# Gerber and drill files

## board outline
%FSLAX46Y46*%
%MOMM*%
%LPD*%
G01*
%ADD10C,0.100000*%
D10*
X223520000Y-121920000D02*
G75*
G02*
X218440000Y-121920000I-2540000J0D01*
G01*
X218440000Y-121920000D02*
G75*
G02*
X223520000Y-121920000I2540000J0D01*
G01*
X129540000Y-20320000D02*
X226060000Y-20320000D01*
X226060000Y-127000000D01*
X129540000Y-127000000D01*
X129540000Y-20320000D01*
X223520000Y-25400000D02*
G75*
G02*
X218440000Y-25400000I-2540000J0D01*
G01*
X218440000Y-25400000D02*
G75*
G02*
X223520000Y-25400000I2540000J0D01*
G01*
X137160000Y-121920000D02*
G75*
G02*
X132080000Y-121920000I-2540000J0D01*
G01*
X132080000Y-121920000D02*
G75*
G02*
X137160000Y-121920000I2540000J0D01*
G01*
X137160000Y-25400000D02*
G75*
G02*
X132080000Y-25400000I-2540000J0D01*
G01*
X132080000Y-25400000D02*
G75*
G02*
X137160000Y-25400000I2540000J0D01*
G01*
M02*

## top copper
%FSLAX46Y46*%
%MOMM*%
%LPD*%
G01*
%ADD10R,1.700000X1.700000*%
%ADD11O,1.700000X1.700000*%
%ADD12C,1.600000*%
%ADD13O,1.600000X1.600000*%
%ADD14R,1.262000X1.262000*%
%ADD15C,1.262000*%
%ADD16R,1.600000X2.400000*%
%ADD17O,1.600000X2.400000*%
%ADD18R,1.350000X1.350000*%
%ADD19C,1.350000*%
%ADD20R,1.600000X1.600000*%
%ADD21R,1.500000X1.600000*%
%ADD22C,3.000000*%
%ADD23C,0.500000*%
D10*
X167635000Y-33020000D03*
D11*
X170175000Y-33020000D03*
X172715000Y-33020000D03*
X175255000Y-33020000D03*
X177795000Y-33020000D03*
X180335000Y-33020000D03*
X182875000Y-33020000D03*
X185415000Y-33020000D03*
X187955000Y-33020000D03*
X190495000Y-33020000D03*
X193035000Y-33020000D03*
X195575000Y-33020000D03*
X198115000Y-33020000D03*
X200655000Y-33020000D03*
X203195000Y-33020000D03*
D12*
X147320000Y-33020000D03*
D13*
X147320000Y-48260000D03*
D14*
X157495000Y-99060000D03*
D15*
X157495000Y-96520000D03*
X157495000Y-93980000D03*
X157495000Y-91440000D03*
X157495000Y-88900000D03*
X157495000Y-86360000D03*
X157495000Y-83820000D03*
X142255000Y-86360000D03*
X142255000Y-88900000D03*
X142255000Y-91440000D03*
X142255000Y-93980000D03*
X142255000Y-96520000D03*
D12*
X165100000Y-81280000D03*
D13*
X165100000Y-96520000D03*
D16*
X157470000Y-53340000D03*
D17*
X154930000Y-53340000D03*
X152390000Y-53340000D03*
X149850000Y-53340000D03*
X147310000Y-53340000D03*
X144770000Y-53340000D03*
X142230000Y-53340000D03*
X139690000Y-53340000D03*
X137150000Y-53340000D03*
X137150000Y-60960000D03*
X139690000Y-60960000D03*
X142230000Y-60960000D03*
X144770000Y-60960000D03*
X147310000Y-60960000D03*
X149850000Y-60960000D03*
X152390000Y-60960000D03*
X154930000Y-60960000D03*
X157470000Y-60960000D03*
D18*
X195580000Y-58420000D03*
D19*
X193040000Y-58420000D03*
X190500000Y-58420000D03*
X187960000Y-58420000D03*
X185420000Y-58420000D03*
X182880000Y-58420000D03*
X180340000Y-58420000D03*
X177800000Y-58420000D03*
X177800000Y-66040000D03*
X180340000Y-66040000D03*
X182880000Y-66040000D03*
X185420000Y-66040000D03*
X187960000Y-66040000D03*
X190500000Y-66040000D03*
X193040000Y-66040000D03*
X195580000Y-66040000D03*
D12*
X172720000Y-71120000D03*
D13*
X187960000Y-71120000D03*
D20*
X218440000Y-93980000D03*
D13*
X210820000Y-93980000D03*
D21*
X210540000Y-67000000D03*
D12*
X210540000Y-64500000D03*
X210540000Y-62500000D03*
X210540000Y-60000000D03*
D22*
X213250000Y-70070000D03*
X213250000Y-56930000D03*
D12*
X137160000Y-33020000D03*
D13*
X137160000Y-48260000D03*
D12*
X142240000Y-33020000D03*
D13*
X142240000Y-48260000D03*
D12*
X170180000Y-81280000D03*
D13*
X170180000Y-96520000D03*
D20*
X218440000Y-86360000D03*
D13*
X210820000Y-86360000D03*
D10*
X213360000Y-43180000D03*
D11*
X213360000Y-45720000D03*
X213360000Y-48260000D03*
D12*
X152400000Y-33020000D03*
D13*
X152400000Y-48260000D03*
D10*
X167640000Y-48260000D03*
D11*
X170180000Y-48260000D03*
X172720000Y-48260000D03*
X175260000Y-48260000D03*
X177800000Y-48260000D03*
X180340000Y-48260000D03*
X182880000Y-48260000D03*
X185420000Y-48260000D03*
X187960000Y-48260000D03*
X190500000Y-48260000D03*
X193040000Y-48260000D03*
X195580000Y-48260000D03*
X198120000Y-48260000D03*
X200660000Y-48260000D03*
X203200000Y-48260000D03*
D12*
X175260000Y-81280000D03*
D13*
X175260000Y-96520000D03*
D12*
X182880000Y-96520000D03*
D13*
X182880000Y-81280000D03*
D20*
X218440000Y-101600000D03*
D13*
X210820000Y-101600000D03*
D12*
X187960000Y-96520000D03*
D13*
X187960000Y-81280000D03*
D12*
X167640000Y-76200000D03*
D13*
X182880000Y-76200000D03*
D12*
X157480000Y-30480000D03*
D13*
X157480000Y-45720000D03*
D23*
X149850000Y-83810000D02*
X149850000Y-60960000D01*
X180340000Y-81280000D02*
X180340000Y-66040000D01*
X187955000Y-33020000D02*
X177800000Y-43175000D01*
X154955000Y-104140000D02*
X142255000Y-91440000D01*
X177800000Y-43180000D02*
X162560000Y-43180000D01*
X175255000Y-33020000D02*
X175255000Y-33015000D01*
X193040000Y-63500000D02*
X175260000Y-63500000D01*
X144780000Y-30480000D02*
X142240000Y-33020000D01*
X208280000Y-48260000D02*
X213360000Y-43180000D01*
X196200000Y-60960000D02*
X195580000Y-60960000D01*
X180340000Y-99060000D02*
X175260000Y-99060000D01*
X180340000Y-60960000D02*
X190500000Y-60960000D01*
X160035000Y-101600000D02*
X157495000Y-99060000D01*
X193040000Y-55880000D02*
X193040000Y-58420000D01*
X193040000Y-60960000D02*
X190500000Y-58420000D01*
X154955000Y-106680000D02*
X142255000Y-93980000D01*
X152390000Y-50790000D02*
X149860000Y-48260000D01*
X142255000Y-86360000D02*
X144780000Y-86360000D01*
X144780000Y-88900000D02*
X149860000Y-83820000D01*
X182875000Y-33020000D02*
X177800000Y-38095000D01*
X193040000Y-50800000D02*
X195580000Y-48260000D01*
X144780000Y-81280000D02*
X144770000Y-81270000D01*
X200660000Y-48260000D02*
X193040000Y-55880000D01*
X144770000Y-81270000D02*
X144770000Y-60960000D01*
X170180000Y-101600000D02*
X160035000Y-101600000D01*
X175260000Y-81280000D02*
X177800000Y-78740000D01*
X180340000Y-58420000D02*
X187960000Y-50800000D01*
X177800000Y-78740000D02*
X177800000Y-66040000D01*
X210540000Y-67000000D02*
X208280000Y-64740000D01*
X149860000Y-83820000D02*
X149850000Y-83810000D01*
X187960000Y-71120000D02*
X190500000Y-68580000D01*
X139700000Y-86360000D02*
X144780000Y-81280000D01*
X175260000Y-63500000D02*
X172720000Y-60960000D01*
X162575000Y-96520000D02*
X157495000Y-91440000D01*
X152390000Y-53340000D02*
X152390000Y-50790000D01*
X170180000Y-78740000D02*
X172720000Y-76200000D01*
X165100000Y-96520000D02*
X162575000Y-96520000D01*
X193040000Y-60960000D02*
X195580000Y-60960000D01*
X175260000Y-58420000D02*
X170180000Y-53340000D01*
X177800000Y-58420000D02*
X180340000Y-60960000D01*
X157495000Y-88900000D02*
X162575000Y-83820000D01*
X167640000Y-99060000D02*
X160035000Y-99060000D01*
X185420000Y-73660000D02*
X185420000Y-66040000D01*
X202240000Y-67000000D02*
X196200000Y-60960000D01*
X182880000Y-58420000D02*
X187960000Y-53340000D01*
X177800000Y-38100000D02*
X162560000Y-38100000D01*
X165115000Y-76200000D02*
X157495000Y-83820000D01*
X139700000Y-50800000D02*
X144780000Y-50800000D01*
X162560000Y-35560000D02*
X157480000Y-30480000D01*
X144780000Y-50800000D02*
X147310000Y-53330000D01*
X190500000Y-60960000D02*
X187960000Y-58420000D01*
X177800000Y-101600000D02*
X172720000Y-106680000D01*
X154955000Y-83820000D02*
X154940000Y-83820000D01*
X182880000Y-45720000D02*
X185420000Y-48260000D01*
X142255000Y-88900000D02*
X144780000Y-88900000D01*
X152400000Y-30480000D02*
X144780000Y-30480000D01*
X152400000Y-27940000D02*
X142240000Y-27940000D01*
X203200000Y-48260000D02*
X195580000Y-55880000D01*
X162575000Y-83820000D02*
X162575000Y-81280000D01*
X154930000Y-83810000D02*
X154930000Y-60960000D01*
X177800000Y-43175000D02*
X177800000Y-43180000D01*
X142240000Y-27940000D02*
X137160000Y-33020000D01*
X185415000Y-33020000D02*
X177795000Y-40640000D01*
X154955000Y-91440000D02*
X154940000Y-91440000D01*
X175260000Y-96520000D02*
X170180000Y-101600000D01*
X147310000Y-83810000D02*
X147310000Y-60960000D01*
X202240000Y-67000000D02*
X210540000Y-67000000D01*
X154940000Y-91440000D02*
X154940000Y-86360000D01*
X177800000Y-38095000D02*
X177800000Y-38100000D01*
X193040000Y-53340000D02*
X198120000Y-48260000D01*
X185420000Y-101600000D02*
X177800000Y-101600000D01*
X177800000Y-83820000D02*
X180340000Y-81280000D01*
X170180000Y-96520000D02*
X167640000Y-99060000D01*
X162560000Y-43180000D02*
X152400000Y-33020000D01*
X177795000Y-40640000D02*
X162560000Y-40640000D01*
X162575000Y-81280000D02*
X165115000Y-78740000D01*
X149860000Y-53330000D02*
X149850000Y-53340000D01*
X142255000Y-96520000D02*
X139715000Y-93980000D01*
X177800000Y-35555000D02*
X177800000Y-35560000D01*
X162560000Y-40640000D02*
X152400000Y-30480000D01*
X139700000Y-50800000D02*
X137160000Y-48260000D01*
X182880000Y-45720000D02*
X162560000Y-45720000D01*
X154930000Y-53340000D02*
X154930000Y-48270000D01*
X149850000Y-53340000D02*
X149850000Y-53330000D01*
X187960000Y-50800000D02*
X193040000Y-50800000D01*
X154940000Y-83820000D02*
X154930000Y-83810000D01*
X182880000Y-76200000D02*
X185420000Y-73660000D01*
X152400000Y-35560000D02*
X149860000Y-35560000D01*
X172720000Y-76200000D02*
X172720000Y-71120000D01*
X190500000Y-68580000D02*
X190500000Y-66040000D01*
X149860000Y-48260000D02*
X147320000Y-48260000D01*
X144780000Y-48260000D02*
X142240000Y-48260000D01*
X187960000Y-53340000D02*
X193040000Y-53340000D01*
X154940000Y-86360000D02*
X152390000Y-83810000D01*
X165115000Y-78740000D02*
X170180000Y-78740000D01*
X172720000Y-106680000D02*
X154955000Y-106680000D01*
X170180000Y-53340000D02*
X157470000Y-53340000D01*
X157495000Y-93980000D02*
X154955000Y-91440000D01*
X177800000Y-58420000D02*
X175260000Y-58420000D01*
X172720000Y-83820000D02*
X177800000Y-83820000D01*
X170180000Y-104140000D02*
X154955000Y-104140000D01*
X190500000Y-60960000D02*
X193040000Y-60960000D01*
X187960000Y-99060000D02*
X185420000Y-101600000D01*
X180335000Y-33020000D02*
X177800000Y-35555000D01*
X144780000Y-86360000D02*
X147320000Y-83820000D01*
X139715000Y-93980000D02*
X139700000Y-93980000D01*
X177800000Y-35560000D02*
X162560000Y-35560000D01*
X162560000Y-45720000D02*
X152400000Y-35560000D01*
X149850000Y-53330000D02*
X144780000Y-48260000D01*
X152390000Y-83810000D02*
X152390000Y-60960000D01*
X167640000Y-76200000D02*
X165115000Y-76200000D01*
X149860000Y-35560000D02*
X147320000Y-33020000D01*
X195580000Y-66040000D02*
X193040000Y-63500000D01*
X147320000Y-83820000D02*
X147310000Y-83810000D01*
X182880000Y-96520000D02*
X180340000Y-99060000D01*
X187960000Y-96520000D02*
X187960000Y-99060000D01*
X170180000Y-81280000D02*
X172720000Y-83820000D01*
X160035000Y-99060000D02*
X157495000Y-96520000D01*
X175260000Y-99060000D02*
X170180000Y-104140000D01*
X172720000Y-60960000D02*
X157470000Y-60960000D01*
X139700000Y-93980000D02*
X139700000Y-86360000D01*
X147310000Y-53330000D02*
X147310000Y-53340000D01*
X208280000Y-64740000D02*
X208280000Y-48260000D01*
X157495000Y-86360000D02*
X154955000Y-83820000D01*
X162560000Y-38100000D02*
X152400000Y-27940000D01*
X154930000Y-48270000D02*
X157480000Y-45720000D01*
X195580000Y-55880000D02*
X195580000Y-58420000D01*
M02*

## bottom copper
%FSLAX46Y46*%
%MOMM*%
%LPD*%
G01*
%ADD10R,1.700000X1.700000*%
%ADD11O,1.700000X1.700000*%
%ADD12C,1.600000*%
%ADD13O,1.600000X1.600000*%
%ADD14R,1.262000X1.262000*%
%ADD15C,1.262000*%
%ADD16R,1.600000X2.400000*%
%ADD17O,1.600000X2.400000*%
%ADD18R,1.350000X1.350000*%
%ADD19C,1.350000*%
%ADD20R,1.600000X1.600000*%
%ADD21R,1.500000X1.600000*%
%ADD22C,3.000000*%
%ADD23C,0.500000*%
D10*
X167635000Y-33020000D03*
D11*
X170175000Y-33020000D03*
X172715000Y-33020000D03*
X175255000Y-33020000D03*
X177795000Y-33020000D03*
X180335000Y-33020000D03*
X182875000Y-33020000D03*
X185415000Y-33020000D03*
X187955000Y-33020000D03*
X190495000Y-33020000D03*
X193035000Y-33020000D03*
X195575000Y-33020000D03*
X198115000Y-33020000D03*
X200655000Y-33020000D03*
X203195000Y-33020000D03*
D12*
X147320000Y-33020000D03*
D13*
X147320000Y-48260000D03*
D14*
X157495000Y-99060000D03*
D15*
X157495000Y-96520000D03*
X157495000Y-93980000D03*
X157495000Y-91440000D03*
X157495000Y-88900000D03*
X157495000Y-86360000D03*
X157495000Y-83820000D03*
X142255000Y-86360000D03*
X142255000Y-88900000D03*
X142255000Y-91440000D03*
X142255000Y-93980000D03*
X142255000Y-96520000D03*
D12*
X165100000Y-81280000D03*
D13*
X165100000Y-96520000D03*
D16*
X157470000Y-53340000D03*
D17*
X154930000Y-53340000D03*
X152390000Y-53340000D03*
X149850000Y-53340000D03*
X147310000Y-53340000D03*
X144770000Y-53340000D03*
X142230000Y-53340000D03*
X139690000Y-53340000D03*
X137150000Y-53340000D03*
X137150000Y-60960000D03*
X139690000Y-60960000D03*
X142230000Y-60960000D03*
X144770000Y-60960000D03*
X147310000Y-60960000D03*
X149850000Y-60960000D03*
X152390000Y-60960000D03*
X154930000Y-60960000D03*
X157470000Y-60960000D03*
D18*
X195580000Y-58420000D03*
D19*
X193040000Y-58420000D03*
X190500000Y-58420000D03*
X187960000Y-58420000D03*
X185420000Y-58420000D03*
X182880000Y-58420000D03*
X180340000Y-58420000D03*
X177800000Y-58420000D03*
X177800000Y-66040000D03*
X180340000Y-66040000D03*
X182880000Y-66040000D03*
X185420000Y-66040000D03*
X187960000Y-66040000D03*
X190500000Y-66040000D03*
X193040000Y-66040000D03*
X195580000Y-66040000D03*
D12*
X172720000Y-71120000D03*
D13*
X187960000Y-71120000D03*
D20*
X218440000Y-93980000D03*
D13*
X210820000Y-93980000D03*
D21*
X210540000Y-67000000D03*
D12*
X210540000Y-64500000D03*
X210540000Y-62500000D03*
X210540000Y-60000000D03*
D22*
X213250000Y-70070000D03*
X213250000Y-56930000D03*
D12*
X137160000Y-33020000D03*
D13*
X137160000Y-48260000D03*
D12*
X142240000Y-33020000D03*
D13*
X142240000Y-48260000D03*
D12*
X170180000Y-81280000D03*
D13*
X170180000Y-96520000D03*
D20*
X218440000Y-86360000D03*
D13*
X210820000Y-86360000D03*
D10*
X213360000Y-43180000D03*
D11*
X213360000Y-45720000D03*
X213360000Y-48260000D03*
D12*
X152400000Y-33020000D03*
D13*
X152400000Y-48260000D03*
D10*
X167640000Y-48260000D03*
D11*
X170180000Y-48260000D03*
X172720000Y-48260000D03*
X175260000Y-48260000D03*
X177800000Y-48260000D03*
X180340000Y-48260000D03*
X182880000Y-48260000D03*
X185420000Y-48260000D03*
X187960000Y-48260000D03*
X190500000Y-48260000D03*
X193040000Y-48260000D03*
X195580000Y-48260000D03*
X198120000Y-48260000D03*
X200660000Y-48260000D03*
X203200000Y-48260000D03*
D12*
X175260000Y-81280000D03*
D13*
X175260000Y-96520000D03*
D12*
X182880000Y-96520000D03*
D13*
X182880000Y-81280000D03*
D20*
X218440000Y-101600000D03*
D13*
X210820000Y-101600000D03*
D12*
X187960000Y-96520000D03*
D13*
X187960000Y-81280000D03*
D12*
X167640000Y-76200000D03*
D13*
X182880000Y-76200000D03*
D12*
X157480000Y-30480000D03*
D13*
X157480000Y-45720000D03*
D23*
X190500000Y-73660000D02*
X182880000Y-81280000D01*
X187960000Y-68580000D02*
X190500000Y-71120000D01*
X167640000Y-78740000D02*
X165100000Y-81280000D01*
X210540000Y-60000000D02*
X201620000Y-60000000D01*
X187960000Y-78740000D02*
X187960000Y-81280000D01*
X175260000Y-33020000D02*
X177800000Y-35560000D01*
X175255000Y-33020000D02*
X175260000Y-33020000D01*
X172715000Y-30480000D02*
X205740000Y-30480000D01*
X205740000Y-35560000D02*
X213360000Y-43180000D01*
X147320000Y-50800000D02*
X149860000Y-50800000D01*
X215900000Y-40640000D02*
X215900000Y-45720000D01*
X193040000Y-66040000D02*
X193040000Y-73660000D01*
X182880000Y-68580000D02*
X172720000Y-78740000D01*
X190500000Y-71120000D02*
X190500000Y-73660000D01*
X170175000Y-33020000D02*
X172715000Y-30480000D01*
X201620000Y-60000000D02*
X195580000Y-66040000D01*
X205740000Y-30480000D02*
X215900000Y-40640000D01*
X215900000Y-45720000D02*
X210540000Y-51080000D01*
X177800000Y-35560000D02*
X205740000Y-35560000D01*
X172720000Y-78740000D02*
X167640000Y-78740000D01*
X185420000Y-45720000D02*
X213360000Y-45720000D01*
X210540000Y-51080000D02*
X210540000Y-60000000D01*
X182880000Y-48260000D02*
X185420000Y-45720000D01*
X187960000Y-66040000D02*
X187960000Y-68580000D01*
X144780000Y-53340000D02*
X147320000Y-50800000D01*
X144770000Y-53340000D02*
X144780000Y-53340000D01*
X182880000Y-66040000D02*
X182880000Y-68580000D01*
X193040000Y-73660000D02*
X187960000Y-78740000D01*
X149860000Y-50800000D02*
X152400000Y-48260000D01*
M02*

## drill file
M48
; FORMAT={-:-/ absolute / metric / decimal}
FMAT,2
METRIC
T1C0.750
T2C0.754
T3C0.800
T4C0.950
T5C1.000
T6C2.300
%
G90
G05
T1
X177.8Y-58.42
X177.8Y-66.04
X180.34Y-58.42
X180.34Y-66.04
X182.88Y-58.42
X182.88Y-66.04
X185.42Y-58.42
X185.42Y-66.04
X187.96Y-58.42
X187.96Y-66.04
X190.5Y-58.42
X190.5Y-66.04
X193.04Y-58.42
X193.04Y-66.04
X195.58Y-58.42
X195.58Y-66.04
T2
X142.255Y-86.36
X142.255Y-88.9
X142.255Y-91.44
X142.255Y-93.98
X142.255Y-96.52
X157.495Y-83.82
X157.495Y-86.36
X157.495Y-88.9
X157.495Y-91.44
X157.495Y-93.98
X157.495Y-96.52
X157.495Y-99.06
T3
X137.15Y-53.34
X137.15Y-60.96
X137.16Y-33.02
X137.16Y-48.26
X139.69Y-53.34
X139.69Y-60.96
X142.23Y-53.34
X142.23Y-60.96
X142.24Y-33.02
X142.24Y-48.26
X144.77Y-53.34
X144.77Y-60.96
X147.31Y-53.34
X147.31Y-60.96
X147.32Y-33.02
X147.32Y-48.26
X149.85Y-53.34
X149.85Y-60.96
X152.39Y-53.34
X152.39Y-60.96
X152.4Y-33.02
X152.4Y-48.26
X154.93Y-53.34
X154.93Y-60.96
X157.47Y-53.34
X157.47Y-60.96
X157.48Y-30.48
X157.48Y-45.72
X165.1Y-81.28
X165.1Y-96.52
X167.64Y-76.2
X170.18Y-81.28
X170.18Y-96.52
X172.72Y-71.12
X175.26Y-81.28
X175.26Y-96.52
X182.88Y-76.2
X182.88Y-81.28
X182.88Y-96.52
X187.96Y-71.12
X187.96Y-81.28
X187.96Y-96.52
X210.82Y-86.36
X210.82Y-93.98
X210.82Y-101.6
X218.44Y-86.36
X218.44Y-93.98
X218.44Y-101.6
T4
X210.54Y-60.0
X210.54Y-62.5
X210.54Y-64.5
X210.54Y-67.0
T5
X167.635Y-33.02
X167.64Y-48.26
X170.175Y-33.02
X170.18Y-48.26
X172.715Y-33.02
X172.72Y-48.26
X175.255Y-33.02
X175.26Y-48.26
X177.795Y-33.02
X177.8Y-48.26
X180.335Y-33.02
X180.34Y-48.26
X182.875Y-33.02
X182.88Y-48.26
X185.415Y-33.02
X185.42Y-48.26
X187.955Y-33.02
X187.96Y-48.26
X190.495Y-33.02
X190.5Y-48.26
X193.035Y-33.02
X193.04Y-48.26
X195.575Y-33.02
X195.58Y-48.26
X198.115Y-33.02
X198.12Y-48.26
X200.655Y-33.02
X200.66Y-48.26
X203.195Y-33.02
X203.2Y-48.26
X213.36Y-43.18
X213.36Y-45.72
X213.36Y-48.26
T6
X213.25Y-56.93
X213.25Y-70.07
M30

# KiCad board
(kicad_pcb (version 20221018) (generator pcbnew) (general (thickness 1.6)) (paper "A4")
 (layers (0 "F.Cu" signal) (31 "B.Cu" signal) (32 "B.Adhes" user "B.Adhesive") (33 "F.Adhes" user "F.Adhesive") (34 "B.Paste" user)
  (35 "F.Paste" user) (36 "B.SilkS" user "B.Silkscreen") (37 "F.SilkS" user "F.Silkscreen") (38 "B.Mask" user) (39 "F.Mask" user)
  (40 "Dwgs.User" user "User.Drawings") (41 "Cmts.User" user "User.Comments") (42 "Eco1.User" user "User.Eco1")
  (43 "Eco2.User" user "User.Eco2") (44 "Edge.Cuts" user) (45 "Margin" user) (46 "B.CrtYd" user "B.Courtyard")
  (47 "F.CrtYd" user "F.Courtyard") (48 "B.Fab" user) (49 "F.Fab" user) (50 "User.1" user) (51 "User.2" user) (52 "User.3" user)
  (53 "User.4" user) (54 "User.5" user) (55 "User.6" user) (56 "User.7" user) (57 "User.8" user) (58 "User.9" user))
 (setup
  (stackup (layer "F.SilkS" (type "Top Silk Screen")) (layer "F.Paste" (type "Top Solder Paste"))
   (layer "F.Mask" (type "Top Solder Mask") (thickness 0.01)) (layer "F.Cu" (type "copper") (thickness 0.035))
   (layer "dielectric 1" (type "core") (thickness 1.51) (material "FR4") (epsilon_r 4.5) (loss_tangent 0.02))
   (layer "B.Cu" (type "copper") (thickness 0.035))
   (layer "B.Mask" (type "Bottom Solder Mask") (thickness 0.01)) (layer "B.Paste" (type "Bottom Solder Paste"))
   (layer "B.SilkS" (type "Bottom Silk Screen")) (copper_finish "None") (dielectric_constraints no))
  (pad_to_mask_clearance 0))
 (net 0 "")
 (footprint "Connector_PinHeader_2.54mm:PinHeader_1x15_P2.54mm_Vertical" (layer "F.Cu") (at 167.635 33.02 90)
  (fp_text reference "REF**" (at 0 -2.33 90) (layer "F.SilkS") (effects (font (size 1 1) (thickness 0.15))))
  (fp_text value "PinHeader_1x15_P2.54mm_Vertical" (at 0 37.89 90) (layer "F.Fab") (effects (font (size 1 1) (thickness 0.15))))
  (pad "1" thru_hole rect (at 0 0 90) (size 1.7 1.7) (drill 1) (layers "*.Cu" "*.Mask"))
  (pad "2" thru_hole oval (at 0 2.54 90) (size 1.7 1.7) (drill 1) (layers "*.Cu" "*.Mask"))
  (pad "3" thru_hole oval (at 0 5.08 90) (size 1.7 1.7) (drill 1) (layers "*.Cu" "*.Mask"))
  (pad "4" thru_hole oval (at 0 7.62 90) (size 1.7 1.7) (drill 1) (layers "*.Cu" "*.Mask"))
  (pad "5" thru_hole oval (at 0 10.16 90) (size 1.7 1.7) (drill 1) (layers "*.Cu" "*.Mask"))
  (pad "6" thru_hole oval (at 0 12.7 90) (size 1.7 1.7) (drill 1) (layers "*.Cu" "*.Mask"))
  (pad "7" thru_hole oval (at 0 15.24 90) (size 1.7 1.7) (drill 1) (layers "*.Cu" "*.Mask"))
  (pad "8" thru_hole oval (at 0 17.78 90) (size 1.7 1.7) (drill 1) (layers "*.Cu" "*.Mask"))
  (pad "9" thru_hole oval (at 0 20.32 90) (size 1.7 1.7) (drill 1) (layers "*.Cu" "*.Mask"))
  (pad "10" thru_hole oval (at 0 22.86 90) (size 1.7 1.7) (drill 1) (layers "*.Cu" "*.Mask"))
  (pad "11" thru_hole oval (at 0 25.4 90) (size 1.7 1.7) (drill 1) (layers "*.Cu" "*.Mask"))
  (pad "12" thru_hole oval (at 0 27.94 90) (size 1.7 1.7) (drill 1) (layers "*.Cu" "*.Mask"))
  (pad "13" thru_hole oval (at 0 30.48 90) (size 1.7 1.7) (drill 1) (layers "*.Cu" "*.Mask"))
  (pad "14" thru_hole oval (at 0 33.02 90) (size 1.7 1.7) (drill 1) (layers "*.Cu" "*.Mask"))
  (pad "15" thru_hole oval (at 0 35.56 90) (size 1.7 1.7) (drill 1) (layers "*.Cu" "*.Mask")))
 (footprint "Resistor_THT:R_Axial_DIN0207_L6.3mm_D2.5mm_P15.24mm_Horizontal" (layer "F.Cu") (at 147.32 33.02 -90)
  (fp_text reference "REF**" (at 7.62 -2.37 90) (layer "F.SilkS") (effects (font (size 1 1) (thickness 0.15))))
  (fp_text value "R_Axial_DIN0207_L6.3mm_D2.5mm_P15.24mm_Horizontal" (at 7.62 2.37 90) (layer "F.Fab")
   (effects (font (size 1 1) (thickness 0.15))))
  (pad "1" thru_hole circle (at 0 0 270) (size 1.6 1.6) (drill 0.8) (layers "*.Cu" "*.Mask"))
  (pad "2" thru_hole oval (at 15.24 0 270) (size 1.6 1.6) (drill 0.8) (layers "*.Cu" "*.Mask")))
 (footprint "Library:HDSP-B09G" (layer "F.Cu") (at 149.875 91.44 90)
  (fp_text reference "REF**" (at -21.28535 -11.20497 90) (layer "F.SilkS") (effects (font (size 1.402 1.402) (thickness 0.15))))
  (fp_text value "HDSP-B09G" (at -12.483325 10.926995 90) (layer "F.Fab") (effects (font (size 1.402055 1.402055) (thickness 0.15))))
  (pad "1" thru_hole rect (at -7.62 7.62 90) (size 1.262 1.262) (drill 0.754) (layers "*.Cu" "*.Mask"))
  (pad "2" thru_hole circle (at -5.08 7.62 90) (size 1.262 1.262) (drill 0.754) (layers "*.Cu" "*.Mask"))
  (pad "3" thru_hole circle (at -2.54 7.62 90) (size 1.262 1.262) (drill 0.754) (layers "*.Cu" "*.Mask"))
  (pad "4" thru_hole circle (at 0 7.62 90) (size 1.262 1.262) (drill 0.754) (layers "*.Cu" "*.Mask"))
  (pad "5" thru_hole circle (at 2.54 7.62 90) (size 1.262 1.262) (drill 0.754) (layers "*.Cu" "*.Mask"))
  (pad "6" thru_hole circle (at 5.08 7.62 90) (size 1.262 1.262) (drill 0.754) (layers "*.Cu" "*.Mask"))
  (pad "7" thru_hole circle (at 7.62 7.62 90) (size 1.262 1.262) (drill 0.754) (layers "*.Cu" "*.Mask"))
  (pad "8" thru_hole circle (at 5.08 -7.62 90) (size 1.262 1.262) (drill 0.754) (layers "*.Cu" "*.Mask"))
  (pad "9" thru_hole circle (at 2.54 -7.62 90) (size 1.262 1.262) (drill 0.754) (layers "*.Cu" "*.Mask"))
  (pad "10" thru_hole circle (at 0 -7.62 90) (size 1.262 1.262) (drill 0.754) (layers "*.Cu" "*.Mask"))
  (pad "11" thru_hole circle (at -2.54 -7.62 90) (size 1.262 1.262) (drill 0.754) (layers "*.Cu" "*.Mask"))
  (pad "12" thru_hole circle (at -5.08 -7.62 90) (size 1.262 1.262) (drill 0.754) (layers "*.Cu" "*.Mask")))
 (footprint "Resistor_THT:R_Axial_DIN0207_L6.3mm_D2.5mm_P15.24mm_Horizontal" (layer "F.Cu") (at 165.1 81.28 -90)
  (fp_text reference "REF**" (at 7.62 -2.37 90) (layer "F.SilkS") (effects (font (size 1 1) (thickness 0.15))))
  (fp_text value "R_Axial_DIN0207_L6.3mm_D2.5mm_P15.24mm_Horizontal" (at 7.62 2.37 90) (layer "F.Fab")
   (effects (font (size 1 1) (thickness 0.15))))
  (pad "1" thru_hole circle (at 0 0 270) (size 1.6 1.6) (drill 0.8) (layers "*.Cu" "*.Mask"))
  (pad "2" thru_hole oval (at 15.24 0 270) (size 1.6 1.6) (drill 0.8) (layers "*.Cu" "*.Mask")))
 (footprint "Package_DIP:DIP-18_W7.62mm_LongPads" (layer "F.Cu") (at 157.47 53.34 -90)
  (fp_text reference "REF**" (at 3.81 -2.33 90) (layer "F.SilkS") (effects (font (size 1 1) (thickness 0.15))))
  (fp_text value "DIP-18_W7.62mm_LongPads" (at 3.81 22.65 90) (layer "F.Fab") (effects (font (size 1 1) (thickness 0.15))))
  (pad "1" thru_hole rect (at 0 0 270) (size 2.4 1.6) (drill 0.8) (layers "*.Cu" "*.Mask"))
  (pad "2" thru_hole oval (at 0 2.54 270) (size 2.4 1.6) (drill 0.8) (layers "*.Cu" "*.Mask"))
  (pad "3" thru_hole oval (at 0 5.08 270) (size 2.4 1.6) (drill 0.8) (layers "*.Cu" "*.Mask"))
  (pad "4" thru_hole oval (at 0 7.62 270) (size 2.4 1.6) (drill 0.8) (layers "*.Cu" "*.Mask"))
  (pad "5" thru_hole oval (at 0 10.16 270) (size 2.4 1.6) (drill 0.8) (layers "*.Cu" "*.Mask"))
  (pad "6" thru_hole oval (at 0 12.7 270) (size 2.4 1.6) (drill 0.8) (layers "*.Cu" "*.Mask"))
  (pad "7" thru_hole oval (at 0 15.24 270) (size 2.4 1.6) (drill 0.8) (layers "*.Cu" "*.Mask"))
  (pad "8" thru_hole oval (at 0 17.78 270) (size 2.4 1.6) (drill 0.8) (layers "*.Cu" "*.Mask"))
  (pad "9" thru_hole oval (at 0 20.32 270) (size 2.4 1.6) (drill 0.8) (layers "*.Cu" "*.Mask"))
  (pad "10" thru_hole oval (at 7.62 20.32 270) (size 2.4 1.6) (drill 0.8) (layers "*.Cu" "*.Mask"))
  (pad "11" thru_hole oval (at 7.62 17.78 270) (size 2.4 1.6) (drill 0.8) (layers "*.Cu" "*.Mask"))
  (pad "12" thru_hole oval (at 7.62 15.24 270) (size 2.4 1.6) (drill 0.8) (layers "*.Cu" "*.Mask"))
  (pad "13" thru_hole oval (at 7.62 12.7 270) (size 2.4 1.6) (drill 0.8) (layers "*.Cu" "*.Mask"))
  (pad "14" thru_hole oval (at 7.62 10.16 270) (size 2.4 1.6) (drill 0.8) (layers "*.Cu" "*.Mask"))
  (pad "15" thru_hole oval (at 7.62 7.62 270) (size 2.4 1.6) (drill 0.8) (layers "*.Cu" "*.Mask"))
  (pad "16" thru_hole oval (at 7.62 5.08 270) (size 2.4 1.6) (drill 0.8) (layers "*.Cu" "*.Mask"))
  (pad "17" thru_hole oval (at 7.62 2.54 270) (size 2.4 1.6) (drill 0.8) (layers "*.Cu" "*.Mask"))
  (pad "18" thru_hole oval (at 7.62 0 270) (size 2.4 1.6) (drill 0.8) (layers "*.Cu" "*.Mask")))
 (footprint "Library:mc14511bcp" (layer "F.Cu") (at 186.69 62.23 -90)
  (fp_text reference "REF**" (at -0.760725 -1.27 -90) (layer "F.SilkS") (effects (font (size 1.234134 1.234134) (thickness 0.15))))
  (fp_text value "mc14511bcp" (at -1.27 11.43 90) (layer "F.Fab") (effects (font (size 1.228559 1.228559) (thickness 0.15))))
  (pad "1" thru_hole rect (at -3.81 -8.89 270) (size 1.35 1.35) (drill 0.75) (layers "*.Cu" "*.Mask"))
  (pad "2" thru_hole circle (at -3.81 -6.35 270) (size 1.35 1.35) (drill 0.75) (layers "*.Cu" "*.Mask"))
  (pad "3" thru_hole circle (at -3.81 -3.81 270) (size 1.35 1.35) (drill 0.75) (layers "*.Cu" "*.Mask"))
  (pad "4" thru_hole circle (at -3.81 -1.27 270) (size 1.35 1.35) (drill 0.75) (layers "*.Cu" "*.Mask"))
  (pad "5" thru_hole circle (at -3.81 1.27 270) (size 1.35 1.35) (drill 0.75) (layers "*.Cu" "*.Mask"))
  (pad "6" thru_hole circle (at -3.81 3.81 270) (size 1.35 1.35) (drill 0.75) (layers "*.Cu" "*.Mask"))
  (pad "7" thru_hole circle (at -3.81 6.35 270) (size 1.35 1.35) (drill 0.75) (layers "*.Cu" "*.Mask"))
  (pad "8" thru_hole circle (at -3.81 8.89 270) (size 1.35 1.35) (drill 0.75) (layers "*.Cu" "*.Mask"))
  (pad "9" thru_hole circle (at 3.81 8.89 270) (size 1.35 1.35) (drill 0.75) (layers "*.Cu" "*.Mask"))
  (pad "10" thru_hole circle (at 3.81 6.35 270) (size 1.35 1.35) (drill 0.75) (layers "*.Cu" "*.Mask"))
  (pad "11" thru_hole circle (at 3.81 3.81 270) (size 1.35 1.35) (drill 0.75) (layers "*.Cu" "*.Mask"))
  (pad "12" thru_hole circle (at 3.81 1.27 270) (size 1.35 1.35) (drill 0.75) (layers "*.Cu" "*.Mask"))
  (pad "13" thru_hole circle (at 3.81 -1.27 270) (size 1.35 1.35) (drill 0.75) (layers "*.Cu" "*.Mask"))
  (pad "14" thru_hole circle (at 3.81 -3.81 270) (size 1.35 1.35) (drill 0.75) (layers "*.Cu" "*.Mask"))
  (pad "15" thru_hole circle (at 3.81 -6.35 270) (size 1.35 1.35) (drill 0.75) (layers "*.Cu" "*.Mask"))
  (pad "16" thru_hole circle (at 3.81 -8.89 270) (size 1.35 1.35) (drill 0.75) (layers "*.Cu" "*.Mask")))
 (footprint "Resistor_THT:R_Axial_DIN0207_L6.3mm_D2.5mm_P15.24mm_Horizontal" (layer "F.Cu") (at 172.72 71.12)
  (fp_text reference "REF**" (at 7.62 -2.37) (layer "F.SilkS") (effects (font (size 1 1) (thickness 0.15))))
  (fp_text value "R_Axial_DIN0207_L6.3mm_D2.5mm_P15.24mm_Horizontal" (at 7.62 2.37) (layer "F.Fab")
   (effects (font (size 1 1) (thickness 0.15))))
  (pad "1" thru_hole circle (at 0 0) (size 1.6 1.6) (drill 0.8) (layers "*.Cu" "*.Mask"))
  (pad "2" thru_hole oval (at 15.24 0) (size 1.6 1.6) (drill 0.8) (layers "*.Cu" "*.Mask")))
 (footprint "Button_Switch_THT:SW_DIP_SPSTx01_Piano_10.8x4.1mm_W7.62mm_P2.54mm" (layer "F.Cu") (at 218.44 93.98 180)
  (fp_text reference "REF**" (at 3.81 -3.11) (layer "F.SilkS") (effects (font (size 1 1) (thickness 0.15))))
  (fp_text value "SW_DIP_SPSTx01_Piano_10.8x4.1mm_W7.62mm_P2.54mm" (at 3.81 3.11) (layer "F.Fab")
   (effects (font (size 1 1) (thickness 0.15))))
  (pad "1" thru_hole rect (at 0 0 180) (size 1.6 1.6) (drill 0.8) (layers "*.Cu" "*.Mask"))
  (pad "2" thru_hole oval (at 7.62 0 180) (size 1.6 1.6) (drill 0.8) (layers "*.Cu" "*.Mask")))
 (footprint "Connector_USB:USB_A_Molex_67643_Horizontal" (layer "F.Cu") (at 210.54 67 90)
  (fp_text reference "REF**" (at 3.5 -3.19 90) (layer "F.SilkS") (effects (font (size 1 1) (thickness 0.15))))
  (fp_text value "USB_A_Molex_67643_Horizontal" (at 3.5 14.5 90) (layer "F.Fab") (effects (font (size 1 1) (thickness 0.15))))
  (pad "1" thru_hole rect (at 0 0 90) (size 1.6 1.5) (drill 0.95) (layers "*.Cu" "*.Mask"))
  (pad "2" thru_hole circle (at 2.5 0 90) (size 1.6 1.6) (drill 0.95) (layers "*.Cu" "*.Mask"))
  (pad "3" thru_hole circle (at 4.5 0 90) (size 1.6 1.6) (drill 0.95) (layers "*.Cu" "*.Mask"))
  (pad "4" thru_hole circle (at 7 0 90) (size 1.6 1.6) (drill 0.95) (layers "*.Cu" "*.Mask"))
  (pad "5" thru_hole circle (at -3.07 2.71 90) (size 3 3) (drill 2.3) (layers "*.Cu" "*.Mask"))
  (pad "5" thru_hole circle (at 10.07 2.71 90) (size 3 3) (drill 2.3) (layers "*.Cu" "*.Mask")))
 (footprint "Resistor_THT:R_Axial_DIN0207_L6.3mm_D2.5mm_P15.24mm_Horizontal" (layer "F.Cu") (at 137.16 33.02 -90)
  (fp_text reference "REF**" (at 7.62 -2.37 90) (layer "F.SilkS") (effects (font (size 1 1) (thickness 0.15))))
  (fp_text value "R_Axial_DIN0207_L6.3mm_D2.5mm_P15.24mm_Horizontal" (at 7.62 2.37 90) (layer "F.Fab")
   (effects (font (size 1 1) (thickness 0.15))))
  (pad "1" thru_hole circle (at 0 0 270) (size 1.6 1.6) (drill 0.8) (layers "*.Cu" "*.Mask"))
  (pad "2" thru_hole oval (at 15.24 0 270) (size 1.6 1.6) (drill 0.8) (layers "*.Cu" "*.Mask")))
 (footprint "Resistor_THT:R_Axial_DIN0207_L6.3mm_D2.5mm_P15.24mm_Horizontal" (layer "F.Cu") (at 142.24 33.02 -90)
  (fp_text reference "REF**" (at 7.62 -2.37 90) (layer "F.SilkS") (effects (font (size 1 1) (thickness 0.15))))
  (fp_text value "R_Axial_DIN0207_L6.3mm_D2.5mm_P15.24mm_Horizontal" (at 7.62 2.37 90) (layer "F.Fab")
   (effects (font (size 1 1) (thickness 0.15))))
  (pad "1" thru_hole circle (at 0 0 270) (size 1.6 1.6) (drill 0.8) (layers "*.Cu" "*.Mask"))
  (pad "2" thru_hole oval (at 15.24 0 270) (size 1.6 1.6) (drill 0.8) (layers "*.Cu" "*.Mask")))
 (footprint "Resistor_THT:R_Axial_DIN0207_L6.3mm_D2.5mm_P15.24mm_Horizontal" (layer "F.Cu") (at 170.18 81.28 -90)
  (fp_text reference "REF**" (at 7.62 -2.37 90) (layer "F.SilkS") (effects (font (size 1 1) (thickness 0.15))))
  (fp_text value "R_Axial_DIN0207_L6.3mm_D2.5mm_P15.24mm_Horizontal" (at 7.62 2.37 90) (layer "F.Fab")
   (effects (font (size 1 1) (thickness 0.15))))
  (pad "1" thru_hole circle (at 0 0 270) (size 1.6 1.6) (drill 0.8) (layers "*.Cu" "*.Mask"))
  (pad "2" thru_hole oval (at 15.24 0 270) (size 1.6 1.6) (drill 0.8) (layers "*.Cu" "*.Mask")))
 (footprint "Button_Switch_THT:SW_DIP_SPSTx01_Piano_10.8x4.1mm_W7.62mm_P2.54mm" (layer "F.Cu") (at 218.44 86.36 180)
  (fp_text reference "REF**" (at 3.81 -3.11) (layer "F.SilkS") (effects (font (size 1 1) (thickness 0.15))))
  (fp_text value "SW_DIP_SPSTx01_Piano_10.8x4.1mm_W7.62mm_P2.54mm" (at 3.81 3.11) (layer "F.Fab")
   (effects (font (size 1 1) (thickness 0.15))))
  (pad "1" thru_hole rect (at 0 0 180) (size 1.6 1.6) (drill 0.8) (layers "*.Cu" "*.Mask"))
  (pad "2" thru_hole oval (at 7.62 0 180) (size 1.6 1.6) (drill 0.8) (layers "*.Cu" "*.Mask")))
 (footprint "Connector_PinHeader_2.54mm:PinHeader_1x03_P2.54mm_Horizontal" (layer "F.Cu") (at 213.36 43.18)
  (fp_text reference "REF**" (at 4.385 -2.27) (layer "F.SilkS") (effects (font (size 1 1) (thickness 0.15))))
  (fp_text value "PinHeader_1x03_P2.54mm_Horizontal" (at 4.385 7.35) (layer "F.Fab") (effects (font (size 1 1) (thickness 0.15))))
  (pad "1" thru_hole rect (at 0 0) (size 1.7 1.7) (drill 1) (layers "*.Cu" "*.Mask"))
  (pad "2" thru_hole oval (at 0 2.54) (size 1.7 1.7) (drill 1) (layers "*.Cu" "*.Mask"))
  (pad "3" thru_hole oval (at 0 5.08) (size 1.7 1.7) (drill 1) (layers "*.Cu" "*.Mask")))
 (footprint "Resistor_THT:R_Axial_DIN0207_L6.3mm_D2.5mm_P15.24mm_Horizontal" (layer "F.Cu") (at 152.4 33.02 -90)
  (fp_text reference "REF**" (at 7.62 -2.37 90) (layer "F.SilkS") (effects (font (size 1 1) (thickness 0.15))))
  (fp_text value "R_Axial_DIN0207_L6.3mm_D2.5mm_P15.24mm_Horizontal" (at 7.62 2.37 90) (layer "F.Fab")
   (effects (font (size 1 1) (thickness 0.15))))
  (pad "1" thru_hole circle (at 0 0 270) (size 1.6 1.6) (drill 0.8) (layers "*.Cu" "*.Mask"))
  (pad "2" thru_hole oval (at 15.24 0 270) (size 1.6 1.6) (drill 0.8) (layers "*.Cu" "*.Mask")))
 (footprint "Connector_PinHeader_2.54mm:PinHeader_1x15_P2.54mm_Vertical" (layer "F.Cu") (at 167.64 48.26 90)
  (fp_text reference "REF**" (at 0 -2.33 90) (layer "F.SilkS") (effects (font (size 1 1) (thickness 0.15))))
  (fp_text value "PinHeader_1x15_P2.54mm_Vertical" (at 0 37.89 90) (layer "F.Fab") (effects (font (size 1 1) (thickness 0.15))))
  (pad "1" thru_hole rect (at 0 0 90) (size 1.7 1.7) (drill 1) (layers "*.Cu" "*.Mask"))
  (pad "2" thru_hole oval (at 0 2.54 90) (size 1.7 1.7) (drill 1) (layers "*.Cu" "*.Mask"))
  (pad "3" thru_hole oval (at 0 5.08 90) (size 1.7 1.7) (drill 1) (layers "*.Cu" "*.Mask"))
  (pad "4" thru_hole oval (at 0 7.62 90) (size 1.7 1.7) (drill 1) (layers "*.Cu" "*.Mask"))
  (pad "5" thru_hole oval (at 0 10.16 90) (size 1.7 1.7) (drill 1) (layers "*.Cu" "*.Mask"))
  (pad "6" thru_hole oval (at 0 12.7 90) (size 1.7 1.7) (drill 1) (layers "*.Cu" "*.Mask"))
  (pad "7" thru_hole oval (at 0 15.24 90) (size 1.7 1.7) (drill 1) (layers "*.Cu" "*.Mask"))
  (pad "8" thru_hole oval (at 0 17.78 90) (size 1.7 1.7) (drill 1) (layers "*.Cu" "*.Mask"))
  (pad "9" thru_hole oval (at 0 20.32 90) (size 1.7 1.7) (drill 1) (layers "*.Cu" "*.Mask"))
  (pad "10" thru_hole oval (at 0 22.86 90) (size 1.7 1.7) (drill 1) (layers "*.Cu" "*.Mask"))
  (pad "11" thru_hole oval (at 0 25.4 90) (size 1.7 1.7) (drill 1) (layers "*.Cu" "*.Mask"))
  (pad "12" thru_hole oval (at 0 27.94 90) (size 1.7 1.7) (drill 1) (layers "*.Cu" "*.Mask"))
  (pad "13" thru_hole oval (at 0 30.48 90) (size 1.7 1.7) (drill 1) (layers "*.Cu" "*.Mask"))
  (pad "14" thru_hole oval (at 0 33.02 90) (size 1.7 1.7) (drill 1) (layers "*.Cu" "*.Mask"))
  (pad "15" thru_hole oval (at 0 35.56 90) (size 1.7 1.7) (drill 1) (layers "*.Cu" "*.Mask")))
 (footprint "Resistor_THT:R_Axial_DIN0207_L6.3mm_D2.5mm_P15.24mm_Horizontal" (layer "F.Cu") (at 175.26 81.28 -90)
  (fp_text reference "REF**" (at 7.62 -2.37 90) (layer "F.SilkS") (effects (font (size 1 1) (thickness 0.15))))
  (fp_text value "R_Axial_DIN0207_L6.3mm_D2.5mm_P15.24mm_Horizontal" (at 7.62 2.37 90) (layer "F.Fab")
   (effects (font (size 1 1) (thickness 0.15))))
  (pad "1" thru_hole circle (at 0 0 270) (size 1.6 1.6) (drill 0.8) (layers "*.Cu" "*.Mask"))
  (pad "2" thru_hole oval (at 15.24 0 270) (size 1.6 1.6) (drill 0.8) (layers "*.Cu" "*.Mask")))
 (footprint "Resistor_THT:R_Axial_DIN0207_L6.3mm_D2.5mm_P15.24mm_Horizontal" (layer "F.Cu") (at 182.88 96.52 90)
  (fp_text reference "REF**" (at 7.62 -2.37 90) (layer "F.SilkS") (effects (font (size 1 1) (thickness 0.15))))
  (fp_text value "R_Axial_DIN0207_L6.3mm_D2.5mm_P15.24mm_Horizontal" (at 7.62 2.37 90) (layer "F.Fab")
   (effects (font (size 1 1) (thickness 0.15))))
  (pad "1" thru_hole circle (at 0 0 90) (size 1.6 1.6) (drill 0.8) (layers "*.Cu" "*.Mask"))
  (pad "2" thru_hole oval (at 15.24 0 90) (size 1.6 1.6) (drill 0.8) (layers "*.Cu" "*.Mask")))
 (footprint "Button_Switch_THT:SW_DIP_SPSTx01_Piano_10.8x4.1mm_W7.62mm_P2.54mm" (layer "F.Cu") (at 218.44 101.6 180)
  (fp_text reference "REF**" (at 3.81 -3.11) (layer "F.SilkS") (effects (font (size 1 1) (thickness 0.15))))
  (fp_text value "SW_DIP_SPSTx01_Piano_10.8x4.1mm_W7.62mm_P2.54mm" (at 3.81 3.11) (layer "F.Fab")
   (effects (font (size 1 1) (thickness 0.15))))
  (pad "1" thru_hole rect (at 0 0 180) (size 1.6 1.6) (drill 0.8) (layers "*.Cu" "*.Mask"))
  (pad "2" thru_hole oval (at 7.62 0 180) (size 1.6 1.6) (drill 0.8) (layers "*.Cu" "*.Mask")))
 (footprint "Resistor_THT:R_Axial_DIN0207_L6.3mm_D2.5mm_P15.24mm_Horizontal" (layer "F.Cu") (at 187.96 96.52 90)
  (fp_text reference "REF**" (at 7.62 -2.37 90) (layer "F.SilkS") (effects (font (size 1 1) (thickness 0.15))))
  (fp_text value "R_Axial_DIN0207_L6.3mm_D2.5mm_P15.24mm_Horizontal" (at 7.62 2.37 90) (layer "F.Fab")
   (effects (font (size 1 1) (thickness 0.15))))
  (pad "1" thru_hole circle (at 0 0 90) (size 1.6 1.6) (drill 0.8) (layers "*.Cu" "*.Mask"))
  (pad "2" thru_hole oval (at 15.24 0 90) (size 1.6 1.6) (drill 0.8) (layers "*.Cu" "*.Mask")))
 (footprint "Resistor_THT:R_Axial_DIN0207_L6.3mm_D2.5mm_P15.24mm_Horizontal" (layer "F.Cu") (at 167.64 76.2)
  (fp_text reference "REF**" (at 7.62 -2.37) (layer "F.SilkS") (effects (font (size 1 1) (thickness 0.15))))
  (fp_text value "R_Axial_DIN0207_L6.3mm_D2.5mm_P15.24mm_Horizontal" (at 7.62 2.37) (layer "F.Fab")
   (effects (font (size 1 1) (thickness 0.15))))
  (pad "1" thru_hole circle (at 0 0) (size 1.6 1.6) (drill 0.8) (layers "*.Cu" "*.Mask"))
  (pad "2" thru_hole oval (at 15.24 0) (size 1.6 1.6) (drill 0.8) (layers "*.Cu" "*.Mask")))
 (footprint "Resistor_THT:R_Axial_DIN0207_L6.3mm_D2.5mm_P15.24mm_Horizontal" (layer "F.Cu") (at 157.48 30.48 -90)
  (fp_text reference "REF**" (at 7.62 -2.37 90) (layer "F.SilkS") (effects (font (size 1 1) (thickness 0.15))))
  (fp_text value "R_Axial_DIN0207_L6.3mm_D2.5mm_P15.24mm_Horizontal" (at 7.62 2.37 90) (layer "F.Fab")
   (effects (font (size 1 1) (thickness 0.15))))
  (pad "1" thru_hole circle (at 0 0 270) (size 1.6 1.6) (drill 0.8) (layers "*.Cu" "*.Mask"))
  (pad "2" thru_hole oval (at 15.24 0 270) (size 1.6 1.6) (drill 0.8) (layers "*.Cu" "*.Mask")))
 (gr_circle (center 220.98 121.92) (end 223.52 121.92) (stroke (width 0.1) (type default)) (fill none) (layer "Edge.Cuts"))
 (gr_rect (start 129.54 20.32) (end 226.06 127) (stroke (width 0.1) (type default)) (fill none) (layer "Edge.Cuts"))
 (gr_circle (center 220.98 25.4) (end 223.52 25.4) (stroke (width 0.1) (type default)) (fill none) (layer "Edge.Cuts"))
 (gr_circle (center 134.62 121.92) (end 137.16 121.92) (stroke (width 0.1) (type default)) (fill none) (layer "Edge.Cuts"))
 (gr_circle (center 134.62 25.4) (end 137.16 25.4) (stroke (width 0.1) (type default)) (fill none) (layer "Edge.Cuts"))
 (segment (start 149.85 83.81) (end 149.85 60.96) (width 0.5) (layer "F.Cu") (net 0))
 (segment (start 180.34 81.28) (end 180.34 66.04) (width 0.5) (layer "F.Cu") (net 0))
 (segment (start 187.955 33.02) (end 177.8 43.175) (width 0.5) (layer "F.Cu") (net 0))
 (segment (start 154.955 104.14) (end 142.255 91.44) (width 0.5) (layer "F.Cu") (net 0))
 (segment (start 177.8 43.18) (end 162.56 43.18) (width 0.5) (layer "F.Cu") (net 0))
 (segment (start 175.255 33.02) (end 175.255 33.015) (width 0.5) (layer "F.Cu") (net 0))
 (segment (start 193.04 63.5) (end 175.26 63.5) (width 0.5) (layer "F.Cu") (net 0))
 (segment (start 144.78 30.48) (end 142.24 33.02) (width 0.5) (layer "F.Cu") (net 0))
 (segment (start 208.28 48.26) (end 213.36 43.18) (width 0.5) (layer "F.Cu") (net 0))
 (segment (start 196.2 60.96) (end 195.58 60.96) (width 0.5) (layer "F.Cu") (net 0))
 (segment (start 180.34 99.06) (end 175.26 99.06) (width 0.5) (layer "F.Cu") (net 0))
 (segment (start 180.34 60.96) (end 190.5 60.96) (width 0.5) (layer "F.Cu") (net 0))
 (segment (start 160.035 101.6) (end 157.495 99.06) (width 0.5) (layer "F.Cu") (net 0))
 (segment (start 193.04 55.88) (end 193.04 58.42) (width 0.5) (layer "F.Cu") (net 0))
 (segment (start 193.04 60.96) (end 190.5 58.42) (width 0.5) (layer "F.Cu") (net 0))
 (segment (start 154.955 106.68) (end 142.255 93.98) (width 0.5) (layer "F.Cu") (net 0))
 (segment (start 152.39 50.79) (end 149.86 48.26) (width 0.5) (layer "F.Cu") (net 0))
 (segment (start 142.255 86.36) (end 144.78 86.36) (width 0.5) (layer "F.Cu") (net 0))
 (segment (start 144.78 88.9) (end 149.86 83.82) (width 0.5) (layer "F.Cu") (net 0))
 (segment (start 182.875 33.02) (end 177.8 38.095) (width 0.5) (layer "F.Cu") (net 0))
 (segment (start 193.04 50.8) (end 195.58 48.26) (width 0.5) (layer "F.Cu") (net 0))
 (segment (start 144.78 81.28) (end 144.77 81.27) (width 0.5) (layer "F.Cu") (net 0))
 (segment (start 200.66 48.26) (end 193.04 55.88) (width 0.5) (layer "F.Cu") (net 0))
 (segment (start 144.77 81.27) (end 144.77 60.96) (width 0.5) (layer "F.Cu") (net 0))
 (segment (start 170.18 101.6) (end 160.035 101.6) (width 0.5) (layer "F.Cu") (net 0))
 (segment (start 175.26 81.28) (end 177.8 78.74) (width 0.5) (layer "F.Cu") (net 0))
 (segment (start 180.34 58.42) (end 187.96 50.8) (width 0.5) (layer "F.Cu") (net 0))
 (segment (start 177.8 78.74) (end 177.8 66.04) (width 0.5) (layer "F.Cu") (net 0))
 (segment (start 210.54 67) (end 208.28 64.74) (width 0.5) (layer "F.Cu") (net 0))
 (segment (start 149.86 83.82) (end 149.85 83.81) (width 0.5) (layer "F.Cu") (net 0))
 (segment (start 187.96 71.12) (end 190.5 68.58) (width 0.5) (layer "F.Cu") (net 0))
 (segment (start 139.7 86.36) (end 144.78 81.28) (width 0.5) (layer "F.Cu") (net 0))
 (segment (start 175.26 63.5) (end 172.72 60.96) (width 0.5) (layer "F.Cu") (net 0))
 (segment (start 162.575 96.52) (end 157.495 91.44) (width 0.5) (layer "F.Cu") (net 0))
 (segment (start 152.39 53.34) (end 152.39 50.79) (width 0.5) (layer "F.Cu") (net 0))
 (segment (start 170.18 78.74) (end 172.72 76.2) (width 0.5) (layer "F.Cu") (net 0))
 (segment (start 165.1 96.52) (end 162.575 96.52) (width 0.5) (layer "F.Cu") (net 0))
 (segment (start 193.04 60.96) (end 195.58 60.96) (width 0.5) (layer "F.Cu") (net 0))
 (segment (start 175.26 58.42) (end 170.18 53.34) (width 0.5) (layer "F.Cu") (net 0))
 (segment (start 177.8 58.42) (end 180.34 60.96) (width 0.5) (layer "F.Cu") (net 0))
 (segment (start 157.495 88.9) (end 162.575 83.82) (width 0.5) (layer "F.Cu") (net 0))
 (segment (start 167.64 99.06) (end 160.035 99.06) (width 0.5) (layer "F.Cu") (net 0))
 (segment (start 185.42 73.66) (end 185.42 66.04) (width 0.5) (layer "F.Cu") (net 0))
 (segment (start 202.24 67) (end 196.2 60.96) (width 0.5) (layer "F.Cu") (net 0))
 (segment (start 182.88 58.42) (end 187.96 53.34) (width 0.5) (layer "F.Cu") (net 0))
 (segment (start 177.8 38.1) (end 162.56 38.1) (width 0.5) (layer "F.Cu") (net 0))
 (segment (start 165.115 76.2) (end 157.495 83.82) (width 0.5) (layer "F.Cu") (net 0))
 (segment (start 139.7 50.8) (end 144.78 50.8) (width 0.5) (layer "F.Cu") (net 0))
 (segment (start 162.56 35.56) (end 157.48 30.48) (width 0.5) (layer "F.Cu") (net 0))
 (segment (start 144.78 50.8) (end 147.31 53.33) (width 0.5) (layer "F.Cu") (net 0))
 (segment (start 190.5 60.96) (end 187.96 58.42) (width 0.5) (layer "F.Cu") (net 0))
 (segment (start 177.8 101.6) (end 172.72 106.68) (width 0.5) (layer "F.Cu") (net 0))
 (segment (start 154.955 83.82) (end 154.94 83.82) (width 0.5) (layer "F.Cu") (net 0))
 (segment (start 182.88 45.72) (end 185.42 48.26) (width 0.5) (layer "F.Cu") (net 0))
 (segment (start 142.255 88.9) (end 144.78 88.9) (width 0.5) (layer "F.Cu") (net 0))
 (segment (start 152.4 30.48) (end 144.78 30.48) (width 0.5) (layer "F.Cu") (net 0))
 (segment (start 152.4 27.94) (end 142.24 27.94) (width 0.5) (layer "F.Cu") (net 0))
 (segment (start 203.2 48.26) (end 195.58 55.88) (width 0.5) (layer "F.Cu") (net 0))
 (segment (start 162.575 83.82) (end 162.575 81.28) (width 0.5) (layer "F.Cu") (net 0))
 (segment (start 154.93 83.81) (end 154.93 60.96) (width 0.5) (layer "F.Cu") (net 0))
 (segment (start 177.8 43.175) (end 177.8 43.18) (width 0.5) (layer "F.Cu") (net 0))
 (segment (start 142.24 27.94) (end 137.16 33.02) (width 0.5) (layer "F.Cu") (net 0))
 (segment (start 185.415 33.02) (end 177.795 40.64) (width 0.5) (layer "F.Cu") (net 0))
 (segment (start 154.955 91.44) (end 154.94 91.44) (width 0.5) (layer "F.Cu") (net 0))
 (segment (start 175.26 96.52) (end 170.18 101.6) (width 0.5) (layer "F.Cu") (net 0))
 (segment (start 147.31 83.81) (end 147.31 60.96) (width 0.5) (layer "F.Cu") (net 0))
 (segment (start 202.24 67) (end 210.54 67) (width 0.5) (layer "F.Cu") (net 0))
 (segment (start 154.94 91.44) (end 154.94 86.36) (width 0.5) (layer "F.Cu") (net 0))
 (segment (start 177.8 38.095) (end 177.8 38.1) (width 0.5) (layer "F.Cu") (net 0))
 (segment (start 193.04 53.34) (end 198.12 48.26) (width 0.5) (layer "F.Cu") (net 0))
 (segment (start 185.42 101.6) (end 177.8 101.6) (width 0.5) (layer "F.Cu") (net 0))
 (segment (start 177.8 83.82) (end 180.34 81.28) (width 0.5) (layer "F.Cu") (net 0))
 (segment (start 170.18 96.52) (end 167.64 99.06) (width 0.5) (layer "F.Cu") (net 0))
 (segment (start 162.56 43.18) (end 152.4 33.02) (width 0.5) (layer "F.Cu") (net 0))
 (segment (start 177.795 40.64) (end 162.56 40.64) (width 0.5) (layer "F.Cu") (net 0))
 (segment (start 162.575 81.28) (end 165.115 78.74) (width 0.5) (layer "F.Cu") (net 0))
 (segment (start 149.86 53.33) (end 149.85 53.34) (width 0.5) (layer "F.Cu") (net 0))
 (segment (start 142.255 96.52) (end 139.715 93.98) (width 0.5) (layer "F.Cu") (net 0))
 (segment (start 177.8 35.555) (end 177.8 35.56) (width 0.5) (layer "F.Cu") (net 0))
 (segment (start 162.56 40.64) (end 152.4 30.48) (width 0.5) (layer "F.Cu") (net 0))
 (segment (start 139.7 50.8) (end 137.16 48.26) (width 0.5) (layer "F.Cu") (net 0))
 (segment (start 182.88 45.72) (end 162.56 45.72) (width 0.5) (layer "F.Cu") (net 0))
 (segment (start 154.93 53.34) (end 154.93 48.27) (width 0.5) (layer "F.Cu") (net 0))
 (segment (start 149.85 53.34) (end 149.85 53.33) (width 0.5) (layer "F.Cu") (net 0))
 (segment (start 187.96 50.8) (end 193.04 50.8) (width 0.5) (layer "F.Cu") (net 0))
 (segment (start 154.94 83.82) (end 154.93 83.81) (width 0.5) (layer "F.Cu") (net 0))
 (segment (start 182.88 76.2) (end 185.42 73.66) (width 0.5) (layer "F.Cu") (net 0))
 (segment (start 152.4 35.56) (end 149.86 35.56) (width 0.5) (layer "F.Cu") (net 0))
 (segment (start 172.72 76.2) (end 172.72 71.12) (width 0.5) (layer "F.Cu") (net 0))
 (segment (start 190.5 68.58) (end 190.5 66.04) (width 0.5) (layer "F.Cu") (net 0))
 (segment (start 149.86 48.26) (end 147.32 48.26) (width 0.5) (layer "F.Cu") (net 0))
 (segment (start 144.78 48.26) (end 142.24 48.26) (width 0.5) (layer "F.Cu") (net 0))
 (segment (start 187.96 53.34) (end 193.04 53.34) (width 0.5) (layer "F.Cu") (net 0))
 (segment (start 154.94 86.36) (end 152.39 83.81) (width 0.5) (layer "F.Cu") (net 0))
 (segment (start 165.115 78.74) (end 170.18 78.74) (width 0.5) (layer "F.Cu") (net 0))
 (segment (start 172.72 106.68) (end 154.955 106.68) (width 0.5) (layer "F.Cu") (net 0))
 (segment (start 170.18 53.34) (end 157.47 53.34) (width 0.5) (layer "F.Cu") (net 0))
 (segment (start 157.495 93.98) (end 154.955 91.44) (width 0.5) (layer "F.Cu") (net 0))
 (segment (start 177.8 58.42) (end 175.26 58.42) (width 0.5) (layer "F.Cu") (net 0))
 (segment (start 172.72 83.82) (end 177.8 83.82) (width 0.5) (layer "F.Cu") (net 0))
 (segment (start 170.18 104.14) (end 154.955 104.14) (width 0.5) (layer "F.Cu") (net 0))
 (segment (start 190.5 60.96) (end 193.04 60.96) (width 0.5) (layer "F.Cu") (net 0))
 (segment (start 187.96 99.06) (end 185.42 101.6) (width 0.5) (layer "F.Cu") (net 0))
 (segment (start 180.335 33.02) (end 177.8 35.555) (width 0.5) (layer "F.Cu") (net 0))
 (segment (start 144.78 86.36) (end 147.32 83.82) (width 0.5) (layer "F.Cu") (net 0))
 (segment (start 139.715 93.98) (end 139.7 93.98) (width 0.5) (layer "F.Cu") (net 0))
 (segment (start 177.8 35.56) (end 162.56 35.56) (width 0.5) (layer "F.Cu") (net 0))
 (segment (start 162.56 45.72) (end 152.4 35.56) (width 0.5) (layer "F.Cu") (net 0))
 (segment (start 149.85 53.33) (end 144.78 48.26) (width 0.5) (layer "F.Cu") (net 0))
 (segment (start 152.39 83.81) (end 152.39 60.96) (width 0.5) (layer "F.Cu") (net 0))
 (segment (start 167.64 76.2) (end 165.115 76.2) (width 0.5) (layer "F.Cu") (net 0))
 (segment (start 149.86 35.56) (end 147.32 33.02) (width 0.5) (layer "F.Cu") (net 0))
 (segment (start 195.58 66.04) (end 193.04 63.5) (width 0.5) (layer "F.Cu") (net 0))
 (segment (start 147.32 83.82) (end 147.31 83.81) (width 0.5) (layer "F.Cu") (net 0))
 (segment (start 182.88 96.52) (end 180.34 99.06) (width 0.5) (layer "F.Cu") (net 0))
 (segment (start 187.96 96.52) (end 187.96 99.06) (width 0.5) (layer "F.Cu") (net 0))
 (segment (start 170.18 81.28) (end 172.72 83.82) (width 0.5) (layer "F.Cu") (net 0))
 (segment (start 160.035 99.06) (end 157.495 96.52) (width 0.5) (layer "F.Cu") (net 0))
 (segment (start 175.26 99.06) (end 170.18 104.14) (width 0.5) (layer "F.Cu") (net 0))
 (segment (start 172.72 60.96) (end 157.47 60.96) (width 0.5) (layer "F.Cu") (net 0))
 (segment (start 139.7 93.98) (end 139.7 86.36) (width 0.5) (layer "F.Cu") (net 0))
 (segment (start 147.31 53.33) (end 147.31 53.34) (width 0.5) (layer "F.Cu") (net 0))
 (segment (start 208.28 64.74) (end 208.28 48.26) (width 0.5) (layer "F.Cu") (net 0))
 (segment (start 157.495 86.36) (end 154.955 83.82) (width 0.5) (layer "F.Cu") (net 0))
 (segment (start 162.56 38.1) (end 152.4 27.94) (width 0.5) (layer "F.Cu") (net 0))
 (segment (start 154.93 48.27) (end 157.48 45.72) (width 0.5) (layer "F.Cu") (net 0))
 (segment (start 195.58 55.88) (end 195.58 58.42) (width 0.5) (layer "F.Cu") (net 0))
 (segment (start 190.5 73.66) (end 182.88 81.28) (width 0.5) (layer "B.Cu") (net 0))
 (segment (start 187.96 68.58) (end 190.5 71.12) (width 0.5) (layer "B.Cu") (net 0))
 (segment (start 167.64 78.74) (end 165.1 81.28) (width 0.5) (layer "B.Cu") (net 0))
 (segment (start 210.54 60) (end 201.62 60) (width 0.5) (layer "B.Cu") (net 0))
 (segment (start 187.96 78.74) (end 187.96 81.28) (width 0.5) (layer "B.Cu") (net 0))
 (segment (start 175.26 33.02) (end 177.8 35.56) (width 0.5) (layer "B.Cu") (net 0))
 (segment (start 175.255 33.02) (end 175.26 33.02) (width 0.5) (layer "B.Cu") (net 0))
 (segment (start 172.715 30.48) (end 205.74 30.48) (width 0.5) (layer "B.Cu") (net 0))
 (segment (start 205.74 35.56) (end 213.36 43.18) (width 0.5) (layer "B.Cu") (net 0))
 (segment (start 147.32 50.8) (end 149.86 50.8) (width 0.5) (layer "B.Cu") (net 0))
 (segment (start 215.9 40.64) (end 215.9 45.72) (width 0.5) (layer "B.Cu") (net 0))
 (segment (start 193.04 66.04) (end 193.04 73.66) (width 0.5) (layer "B.Cu") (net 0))
 (segment (start 182.88 68.58) (end 172.72 78.74) (width 0.5) (layer "B.Cu") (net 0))
 (segment (start 190.5 71.12) (end 190.5 73.66) (width 0.5) (layer "B.Cu") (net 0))
 (segment (start 170.175 33.02) (end 172.715 30.48) (width 0.5) (layer "B.Cu") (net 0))
 (segment (start 201.62 60) (end 195.58 66.04) (width 0.5) (layer "B.Cu") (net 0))
 (segment (start 205.74 30.48) (end 215.9 40.64) (width 0.5) (layer "B.Cu") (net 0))
 (segment (start 215.9 45.72) (end 210.54 51.08) (width 0.5) (layer "B.Cu") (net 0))
 (segment (start 177.8 35.56) (end 205.74 35.56) (width 0.5) (layer "B.Cu") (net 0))
 (segment (start 172.72 78.74) (end 167.64 78.74) (width 0.5) (layer "B.Cu") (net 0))
 (segment (start 185.42 45.72) (end 213.36 45.72) (width 0.5) (layer "B.Cu") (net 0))
 (segment (start 210.54 51.08) (end 210.54 60) (width 0.5) (layer "B.Cu") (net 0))
 (segment (start 182.88 48.26) (end 185.42 45.72) (width 0.5) (layer "B.Cu") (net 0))
 (segment (start 187.96 66.04) (end 187.96 68.58) (width 0.5) (layer "B.Cu") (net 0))
 (segment (start 144.78 53.34) (end 147.32 50.8) (width 0.5) (layer "B.Cu") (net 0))
 (segment (start 144.77 53.34) (end 144.78 53.34) (width 0.5) (layer "B.Cu") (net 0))
 (segment (start 182.88 66.04) (end 182.88 68.58) (width 0.5) (layer "B.Cu") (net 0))
 (segment (start 193.04 73.66) (end 187.96 78.74) (width 0.5) (layer "B.Cu") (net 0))
 (segment (start 149.86 50.8) (end 152.4 48.26) (width 0.5) (layer "B.Cu") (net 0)))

